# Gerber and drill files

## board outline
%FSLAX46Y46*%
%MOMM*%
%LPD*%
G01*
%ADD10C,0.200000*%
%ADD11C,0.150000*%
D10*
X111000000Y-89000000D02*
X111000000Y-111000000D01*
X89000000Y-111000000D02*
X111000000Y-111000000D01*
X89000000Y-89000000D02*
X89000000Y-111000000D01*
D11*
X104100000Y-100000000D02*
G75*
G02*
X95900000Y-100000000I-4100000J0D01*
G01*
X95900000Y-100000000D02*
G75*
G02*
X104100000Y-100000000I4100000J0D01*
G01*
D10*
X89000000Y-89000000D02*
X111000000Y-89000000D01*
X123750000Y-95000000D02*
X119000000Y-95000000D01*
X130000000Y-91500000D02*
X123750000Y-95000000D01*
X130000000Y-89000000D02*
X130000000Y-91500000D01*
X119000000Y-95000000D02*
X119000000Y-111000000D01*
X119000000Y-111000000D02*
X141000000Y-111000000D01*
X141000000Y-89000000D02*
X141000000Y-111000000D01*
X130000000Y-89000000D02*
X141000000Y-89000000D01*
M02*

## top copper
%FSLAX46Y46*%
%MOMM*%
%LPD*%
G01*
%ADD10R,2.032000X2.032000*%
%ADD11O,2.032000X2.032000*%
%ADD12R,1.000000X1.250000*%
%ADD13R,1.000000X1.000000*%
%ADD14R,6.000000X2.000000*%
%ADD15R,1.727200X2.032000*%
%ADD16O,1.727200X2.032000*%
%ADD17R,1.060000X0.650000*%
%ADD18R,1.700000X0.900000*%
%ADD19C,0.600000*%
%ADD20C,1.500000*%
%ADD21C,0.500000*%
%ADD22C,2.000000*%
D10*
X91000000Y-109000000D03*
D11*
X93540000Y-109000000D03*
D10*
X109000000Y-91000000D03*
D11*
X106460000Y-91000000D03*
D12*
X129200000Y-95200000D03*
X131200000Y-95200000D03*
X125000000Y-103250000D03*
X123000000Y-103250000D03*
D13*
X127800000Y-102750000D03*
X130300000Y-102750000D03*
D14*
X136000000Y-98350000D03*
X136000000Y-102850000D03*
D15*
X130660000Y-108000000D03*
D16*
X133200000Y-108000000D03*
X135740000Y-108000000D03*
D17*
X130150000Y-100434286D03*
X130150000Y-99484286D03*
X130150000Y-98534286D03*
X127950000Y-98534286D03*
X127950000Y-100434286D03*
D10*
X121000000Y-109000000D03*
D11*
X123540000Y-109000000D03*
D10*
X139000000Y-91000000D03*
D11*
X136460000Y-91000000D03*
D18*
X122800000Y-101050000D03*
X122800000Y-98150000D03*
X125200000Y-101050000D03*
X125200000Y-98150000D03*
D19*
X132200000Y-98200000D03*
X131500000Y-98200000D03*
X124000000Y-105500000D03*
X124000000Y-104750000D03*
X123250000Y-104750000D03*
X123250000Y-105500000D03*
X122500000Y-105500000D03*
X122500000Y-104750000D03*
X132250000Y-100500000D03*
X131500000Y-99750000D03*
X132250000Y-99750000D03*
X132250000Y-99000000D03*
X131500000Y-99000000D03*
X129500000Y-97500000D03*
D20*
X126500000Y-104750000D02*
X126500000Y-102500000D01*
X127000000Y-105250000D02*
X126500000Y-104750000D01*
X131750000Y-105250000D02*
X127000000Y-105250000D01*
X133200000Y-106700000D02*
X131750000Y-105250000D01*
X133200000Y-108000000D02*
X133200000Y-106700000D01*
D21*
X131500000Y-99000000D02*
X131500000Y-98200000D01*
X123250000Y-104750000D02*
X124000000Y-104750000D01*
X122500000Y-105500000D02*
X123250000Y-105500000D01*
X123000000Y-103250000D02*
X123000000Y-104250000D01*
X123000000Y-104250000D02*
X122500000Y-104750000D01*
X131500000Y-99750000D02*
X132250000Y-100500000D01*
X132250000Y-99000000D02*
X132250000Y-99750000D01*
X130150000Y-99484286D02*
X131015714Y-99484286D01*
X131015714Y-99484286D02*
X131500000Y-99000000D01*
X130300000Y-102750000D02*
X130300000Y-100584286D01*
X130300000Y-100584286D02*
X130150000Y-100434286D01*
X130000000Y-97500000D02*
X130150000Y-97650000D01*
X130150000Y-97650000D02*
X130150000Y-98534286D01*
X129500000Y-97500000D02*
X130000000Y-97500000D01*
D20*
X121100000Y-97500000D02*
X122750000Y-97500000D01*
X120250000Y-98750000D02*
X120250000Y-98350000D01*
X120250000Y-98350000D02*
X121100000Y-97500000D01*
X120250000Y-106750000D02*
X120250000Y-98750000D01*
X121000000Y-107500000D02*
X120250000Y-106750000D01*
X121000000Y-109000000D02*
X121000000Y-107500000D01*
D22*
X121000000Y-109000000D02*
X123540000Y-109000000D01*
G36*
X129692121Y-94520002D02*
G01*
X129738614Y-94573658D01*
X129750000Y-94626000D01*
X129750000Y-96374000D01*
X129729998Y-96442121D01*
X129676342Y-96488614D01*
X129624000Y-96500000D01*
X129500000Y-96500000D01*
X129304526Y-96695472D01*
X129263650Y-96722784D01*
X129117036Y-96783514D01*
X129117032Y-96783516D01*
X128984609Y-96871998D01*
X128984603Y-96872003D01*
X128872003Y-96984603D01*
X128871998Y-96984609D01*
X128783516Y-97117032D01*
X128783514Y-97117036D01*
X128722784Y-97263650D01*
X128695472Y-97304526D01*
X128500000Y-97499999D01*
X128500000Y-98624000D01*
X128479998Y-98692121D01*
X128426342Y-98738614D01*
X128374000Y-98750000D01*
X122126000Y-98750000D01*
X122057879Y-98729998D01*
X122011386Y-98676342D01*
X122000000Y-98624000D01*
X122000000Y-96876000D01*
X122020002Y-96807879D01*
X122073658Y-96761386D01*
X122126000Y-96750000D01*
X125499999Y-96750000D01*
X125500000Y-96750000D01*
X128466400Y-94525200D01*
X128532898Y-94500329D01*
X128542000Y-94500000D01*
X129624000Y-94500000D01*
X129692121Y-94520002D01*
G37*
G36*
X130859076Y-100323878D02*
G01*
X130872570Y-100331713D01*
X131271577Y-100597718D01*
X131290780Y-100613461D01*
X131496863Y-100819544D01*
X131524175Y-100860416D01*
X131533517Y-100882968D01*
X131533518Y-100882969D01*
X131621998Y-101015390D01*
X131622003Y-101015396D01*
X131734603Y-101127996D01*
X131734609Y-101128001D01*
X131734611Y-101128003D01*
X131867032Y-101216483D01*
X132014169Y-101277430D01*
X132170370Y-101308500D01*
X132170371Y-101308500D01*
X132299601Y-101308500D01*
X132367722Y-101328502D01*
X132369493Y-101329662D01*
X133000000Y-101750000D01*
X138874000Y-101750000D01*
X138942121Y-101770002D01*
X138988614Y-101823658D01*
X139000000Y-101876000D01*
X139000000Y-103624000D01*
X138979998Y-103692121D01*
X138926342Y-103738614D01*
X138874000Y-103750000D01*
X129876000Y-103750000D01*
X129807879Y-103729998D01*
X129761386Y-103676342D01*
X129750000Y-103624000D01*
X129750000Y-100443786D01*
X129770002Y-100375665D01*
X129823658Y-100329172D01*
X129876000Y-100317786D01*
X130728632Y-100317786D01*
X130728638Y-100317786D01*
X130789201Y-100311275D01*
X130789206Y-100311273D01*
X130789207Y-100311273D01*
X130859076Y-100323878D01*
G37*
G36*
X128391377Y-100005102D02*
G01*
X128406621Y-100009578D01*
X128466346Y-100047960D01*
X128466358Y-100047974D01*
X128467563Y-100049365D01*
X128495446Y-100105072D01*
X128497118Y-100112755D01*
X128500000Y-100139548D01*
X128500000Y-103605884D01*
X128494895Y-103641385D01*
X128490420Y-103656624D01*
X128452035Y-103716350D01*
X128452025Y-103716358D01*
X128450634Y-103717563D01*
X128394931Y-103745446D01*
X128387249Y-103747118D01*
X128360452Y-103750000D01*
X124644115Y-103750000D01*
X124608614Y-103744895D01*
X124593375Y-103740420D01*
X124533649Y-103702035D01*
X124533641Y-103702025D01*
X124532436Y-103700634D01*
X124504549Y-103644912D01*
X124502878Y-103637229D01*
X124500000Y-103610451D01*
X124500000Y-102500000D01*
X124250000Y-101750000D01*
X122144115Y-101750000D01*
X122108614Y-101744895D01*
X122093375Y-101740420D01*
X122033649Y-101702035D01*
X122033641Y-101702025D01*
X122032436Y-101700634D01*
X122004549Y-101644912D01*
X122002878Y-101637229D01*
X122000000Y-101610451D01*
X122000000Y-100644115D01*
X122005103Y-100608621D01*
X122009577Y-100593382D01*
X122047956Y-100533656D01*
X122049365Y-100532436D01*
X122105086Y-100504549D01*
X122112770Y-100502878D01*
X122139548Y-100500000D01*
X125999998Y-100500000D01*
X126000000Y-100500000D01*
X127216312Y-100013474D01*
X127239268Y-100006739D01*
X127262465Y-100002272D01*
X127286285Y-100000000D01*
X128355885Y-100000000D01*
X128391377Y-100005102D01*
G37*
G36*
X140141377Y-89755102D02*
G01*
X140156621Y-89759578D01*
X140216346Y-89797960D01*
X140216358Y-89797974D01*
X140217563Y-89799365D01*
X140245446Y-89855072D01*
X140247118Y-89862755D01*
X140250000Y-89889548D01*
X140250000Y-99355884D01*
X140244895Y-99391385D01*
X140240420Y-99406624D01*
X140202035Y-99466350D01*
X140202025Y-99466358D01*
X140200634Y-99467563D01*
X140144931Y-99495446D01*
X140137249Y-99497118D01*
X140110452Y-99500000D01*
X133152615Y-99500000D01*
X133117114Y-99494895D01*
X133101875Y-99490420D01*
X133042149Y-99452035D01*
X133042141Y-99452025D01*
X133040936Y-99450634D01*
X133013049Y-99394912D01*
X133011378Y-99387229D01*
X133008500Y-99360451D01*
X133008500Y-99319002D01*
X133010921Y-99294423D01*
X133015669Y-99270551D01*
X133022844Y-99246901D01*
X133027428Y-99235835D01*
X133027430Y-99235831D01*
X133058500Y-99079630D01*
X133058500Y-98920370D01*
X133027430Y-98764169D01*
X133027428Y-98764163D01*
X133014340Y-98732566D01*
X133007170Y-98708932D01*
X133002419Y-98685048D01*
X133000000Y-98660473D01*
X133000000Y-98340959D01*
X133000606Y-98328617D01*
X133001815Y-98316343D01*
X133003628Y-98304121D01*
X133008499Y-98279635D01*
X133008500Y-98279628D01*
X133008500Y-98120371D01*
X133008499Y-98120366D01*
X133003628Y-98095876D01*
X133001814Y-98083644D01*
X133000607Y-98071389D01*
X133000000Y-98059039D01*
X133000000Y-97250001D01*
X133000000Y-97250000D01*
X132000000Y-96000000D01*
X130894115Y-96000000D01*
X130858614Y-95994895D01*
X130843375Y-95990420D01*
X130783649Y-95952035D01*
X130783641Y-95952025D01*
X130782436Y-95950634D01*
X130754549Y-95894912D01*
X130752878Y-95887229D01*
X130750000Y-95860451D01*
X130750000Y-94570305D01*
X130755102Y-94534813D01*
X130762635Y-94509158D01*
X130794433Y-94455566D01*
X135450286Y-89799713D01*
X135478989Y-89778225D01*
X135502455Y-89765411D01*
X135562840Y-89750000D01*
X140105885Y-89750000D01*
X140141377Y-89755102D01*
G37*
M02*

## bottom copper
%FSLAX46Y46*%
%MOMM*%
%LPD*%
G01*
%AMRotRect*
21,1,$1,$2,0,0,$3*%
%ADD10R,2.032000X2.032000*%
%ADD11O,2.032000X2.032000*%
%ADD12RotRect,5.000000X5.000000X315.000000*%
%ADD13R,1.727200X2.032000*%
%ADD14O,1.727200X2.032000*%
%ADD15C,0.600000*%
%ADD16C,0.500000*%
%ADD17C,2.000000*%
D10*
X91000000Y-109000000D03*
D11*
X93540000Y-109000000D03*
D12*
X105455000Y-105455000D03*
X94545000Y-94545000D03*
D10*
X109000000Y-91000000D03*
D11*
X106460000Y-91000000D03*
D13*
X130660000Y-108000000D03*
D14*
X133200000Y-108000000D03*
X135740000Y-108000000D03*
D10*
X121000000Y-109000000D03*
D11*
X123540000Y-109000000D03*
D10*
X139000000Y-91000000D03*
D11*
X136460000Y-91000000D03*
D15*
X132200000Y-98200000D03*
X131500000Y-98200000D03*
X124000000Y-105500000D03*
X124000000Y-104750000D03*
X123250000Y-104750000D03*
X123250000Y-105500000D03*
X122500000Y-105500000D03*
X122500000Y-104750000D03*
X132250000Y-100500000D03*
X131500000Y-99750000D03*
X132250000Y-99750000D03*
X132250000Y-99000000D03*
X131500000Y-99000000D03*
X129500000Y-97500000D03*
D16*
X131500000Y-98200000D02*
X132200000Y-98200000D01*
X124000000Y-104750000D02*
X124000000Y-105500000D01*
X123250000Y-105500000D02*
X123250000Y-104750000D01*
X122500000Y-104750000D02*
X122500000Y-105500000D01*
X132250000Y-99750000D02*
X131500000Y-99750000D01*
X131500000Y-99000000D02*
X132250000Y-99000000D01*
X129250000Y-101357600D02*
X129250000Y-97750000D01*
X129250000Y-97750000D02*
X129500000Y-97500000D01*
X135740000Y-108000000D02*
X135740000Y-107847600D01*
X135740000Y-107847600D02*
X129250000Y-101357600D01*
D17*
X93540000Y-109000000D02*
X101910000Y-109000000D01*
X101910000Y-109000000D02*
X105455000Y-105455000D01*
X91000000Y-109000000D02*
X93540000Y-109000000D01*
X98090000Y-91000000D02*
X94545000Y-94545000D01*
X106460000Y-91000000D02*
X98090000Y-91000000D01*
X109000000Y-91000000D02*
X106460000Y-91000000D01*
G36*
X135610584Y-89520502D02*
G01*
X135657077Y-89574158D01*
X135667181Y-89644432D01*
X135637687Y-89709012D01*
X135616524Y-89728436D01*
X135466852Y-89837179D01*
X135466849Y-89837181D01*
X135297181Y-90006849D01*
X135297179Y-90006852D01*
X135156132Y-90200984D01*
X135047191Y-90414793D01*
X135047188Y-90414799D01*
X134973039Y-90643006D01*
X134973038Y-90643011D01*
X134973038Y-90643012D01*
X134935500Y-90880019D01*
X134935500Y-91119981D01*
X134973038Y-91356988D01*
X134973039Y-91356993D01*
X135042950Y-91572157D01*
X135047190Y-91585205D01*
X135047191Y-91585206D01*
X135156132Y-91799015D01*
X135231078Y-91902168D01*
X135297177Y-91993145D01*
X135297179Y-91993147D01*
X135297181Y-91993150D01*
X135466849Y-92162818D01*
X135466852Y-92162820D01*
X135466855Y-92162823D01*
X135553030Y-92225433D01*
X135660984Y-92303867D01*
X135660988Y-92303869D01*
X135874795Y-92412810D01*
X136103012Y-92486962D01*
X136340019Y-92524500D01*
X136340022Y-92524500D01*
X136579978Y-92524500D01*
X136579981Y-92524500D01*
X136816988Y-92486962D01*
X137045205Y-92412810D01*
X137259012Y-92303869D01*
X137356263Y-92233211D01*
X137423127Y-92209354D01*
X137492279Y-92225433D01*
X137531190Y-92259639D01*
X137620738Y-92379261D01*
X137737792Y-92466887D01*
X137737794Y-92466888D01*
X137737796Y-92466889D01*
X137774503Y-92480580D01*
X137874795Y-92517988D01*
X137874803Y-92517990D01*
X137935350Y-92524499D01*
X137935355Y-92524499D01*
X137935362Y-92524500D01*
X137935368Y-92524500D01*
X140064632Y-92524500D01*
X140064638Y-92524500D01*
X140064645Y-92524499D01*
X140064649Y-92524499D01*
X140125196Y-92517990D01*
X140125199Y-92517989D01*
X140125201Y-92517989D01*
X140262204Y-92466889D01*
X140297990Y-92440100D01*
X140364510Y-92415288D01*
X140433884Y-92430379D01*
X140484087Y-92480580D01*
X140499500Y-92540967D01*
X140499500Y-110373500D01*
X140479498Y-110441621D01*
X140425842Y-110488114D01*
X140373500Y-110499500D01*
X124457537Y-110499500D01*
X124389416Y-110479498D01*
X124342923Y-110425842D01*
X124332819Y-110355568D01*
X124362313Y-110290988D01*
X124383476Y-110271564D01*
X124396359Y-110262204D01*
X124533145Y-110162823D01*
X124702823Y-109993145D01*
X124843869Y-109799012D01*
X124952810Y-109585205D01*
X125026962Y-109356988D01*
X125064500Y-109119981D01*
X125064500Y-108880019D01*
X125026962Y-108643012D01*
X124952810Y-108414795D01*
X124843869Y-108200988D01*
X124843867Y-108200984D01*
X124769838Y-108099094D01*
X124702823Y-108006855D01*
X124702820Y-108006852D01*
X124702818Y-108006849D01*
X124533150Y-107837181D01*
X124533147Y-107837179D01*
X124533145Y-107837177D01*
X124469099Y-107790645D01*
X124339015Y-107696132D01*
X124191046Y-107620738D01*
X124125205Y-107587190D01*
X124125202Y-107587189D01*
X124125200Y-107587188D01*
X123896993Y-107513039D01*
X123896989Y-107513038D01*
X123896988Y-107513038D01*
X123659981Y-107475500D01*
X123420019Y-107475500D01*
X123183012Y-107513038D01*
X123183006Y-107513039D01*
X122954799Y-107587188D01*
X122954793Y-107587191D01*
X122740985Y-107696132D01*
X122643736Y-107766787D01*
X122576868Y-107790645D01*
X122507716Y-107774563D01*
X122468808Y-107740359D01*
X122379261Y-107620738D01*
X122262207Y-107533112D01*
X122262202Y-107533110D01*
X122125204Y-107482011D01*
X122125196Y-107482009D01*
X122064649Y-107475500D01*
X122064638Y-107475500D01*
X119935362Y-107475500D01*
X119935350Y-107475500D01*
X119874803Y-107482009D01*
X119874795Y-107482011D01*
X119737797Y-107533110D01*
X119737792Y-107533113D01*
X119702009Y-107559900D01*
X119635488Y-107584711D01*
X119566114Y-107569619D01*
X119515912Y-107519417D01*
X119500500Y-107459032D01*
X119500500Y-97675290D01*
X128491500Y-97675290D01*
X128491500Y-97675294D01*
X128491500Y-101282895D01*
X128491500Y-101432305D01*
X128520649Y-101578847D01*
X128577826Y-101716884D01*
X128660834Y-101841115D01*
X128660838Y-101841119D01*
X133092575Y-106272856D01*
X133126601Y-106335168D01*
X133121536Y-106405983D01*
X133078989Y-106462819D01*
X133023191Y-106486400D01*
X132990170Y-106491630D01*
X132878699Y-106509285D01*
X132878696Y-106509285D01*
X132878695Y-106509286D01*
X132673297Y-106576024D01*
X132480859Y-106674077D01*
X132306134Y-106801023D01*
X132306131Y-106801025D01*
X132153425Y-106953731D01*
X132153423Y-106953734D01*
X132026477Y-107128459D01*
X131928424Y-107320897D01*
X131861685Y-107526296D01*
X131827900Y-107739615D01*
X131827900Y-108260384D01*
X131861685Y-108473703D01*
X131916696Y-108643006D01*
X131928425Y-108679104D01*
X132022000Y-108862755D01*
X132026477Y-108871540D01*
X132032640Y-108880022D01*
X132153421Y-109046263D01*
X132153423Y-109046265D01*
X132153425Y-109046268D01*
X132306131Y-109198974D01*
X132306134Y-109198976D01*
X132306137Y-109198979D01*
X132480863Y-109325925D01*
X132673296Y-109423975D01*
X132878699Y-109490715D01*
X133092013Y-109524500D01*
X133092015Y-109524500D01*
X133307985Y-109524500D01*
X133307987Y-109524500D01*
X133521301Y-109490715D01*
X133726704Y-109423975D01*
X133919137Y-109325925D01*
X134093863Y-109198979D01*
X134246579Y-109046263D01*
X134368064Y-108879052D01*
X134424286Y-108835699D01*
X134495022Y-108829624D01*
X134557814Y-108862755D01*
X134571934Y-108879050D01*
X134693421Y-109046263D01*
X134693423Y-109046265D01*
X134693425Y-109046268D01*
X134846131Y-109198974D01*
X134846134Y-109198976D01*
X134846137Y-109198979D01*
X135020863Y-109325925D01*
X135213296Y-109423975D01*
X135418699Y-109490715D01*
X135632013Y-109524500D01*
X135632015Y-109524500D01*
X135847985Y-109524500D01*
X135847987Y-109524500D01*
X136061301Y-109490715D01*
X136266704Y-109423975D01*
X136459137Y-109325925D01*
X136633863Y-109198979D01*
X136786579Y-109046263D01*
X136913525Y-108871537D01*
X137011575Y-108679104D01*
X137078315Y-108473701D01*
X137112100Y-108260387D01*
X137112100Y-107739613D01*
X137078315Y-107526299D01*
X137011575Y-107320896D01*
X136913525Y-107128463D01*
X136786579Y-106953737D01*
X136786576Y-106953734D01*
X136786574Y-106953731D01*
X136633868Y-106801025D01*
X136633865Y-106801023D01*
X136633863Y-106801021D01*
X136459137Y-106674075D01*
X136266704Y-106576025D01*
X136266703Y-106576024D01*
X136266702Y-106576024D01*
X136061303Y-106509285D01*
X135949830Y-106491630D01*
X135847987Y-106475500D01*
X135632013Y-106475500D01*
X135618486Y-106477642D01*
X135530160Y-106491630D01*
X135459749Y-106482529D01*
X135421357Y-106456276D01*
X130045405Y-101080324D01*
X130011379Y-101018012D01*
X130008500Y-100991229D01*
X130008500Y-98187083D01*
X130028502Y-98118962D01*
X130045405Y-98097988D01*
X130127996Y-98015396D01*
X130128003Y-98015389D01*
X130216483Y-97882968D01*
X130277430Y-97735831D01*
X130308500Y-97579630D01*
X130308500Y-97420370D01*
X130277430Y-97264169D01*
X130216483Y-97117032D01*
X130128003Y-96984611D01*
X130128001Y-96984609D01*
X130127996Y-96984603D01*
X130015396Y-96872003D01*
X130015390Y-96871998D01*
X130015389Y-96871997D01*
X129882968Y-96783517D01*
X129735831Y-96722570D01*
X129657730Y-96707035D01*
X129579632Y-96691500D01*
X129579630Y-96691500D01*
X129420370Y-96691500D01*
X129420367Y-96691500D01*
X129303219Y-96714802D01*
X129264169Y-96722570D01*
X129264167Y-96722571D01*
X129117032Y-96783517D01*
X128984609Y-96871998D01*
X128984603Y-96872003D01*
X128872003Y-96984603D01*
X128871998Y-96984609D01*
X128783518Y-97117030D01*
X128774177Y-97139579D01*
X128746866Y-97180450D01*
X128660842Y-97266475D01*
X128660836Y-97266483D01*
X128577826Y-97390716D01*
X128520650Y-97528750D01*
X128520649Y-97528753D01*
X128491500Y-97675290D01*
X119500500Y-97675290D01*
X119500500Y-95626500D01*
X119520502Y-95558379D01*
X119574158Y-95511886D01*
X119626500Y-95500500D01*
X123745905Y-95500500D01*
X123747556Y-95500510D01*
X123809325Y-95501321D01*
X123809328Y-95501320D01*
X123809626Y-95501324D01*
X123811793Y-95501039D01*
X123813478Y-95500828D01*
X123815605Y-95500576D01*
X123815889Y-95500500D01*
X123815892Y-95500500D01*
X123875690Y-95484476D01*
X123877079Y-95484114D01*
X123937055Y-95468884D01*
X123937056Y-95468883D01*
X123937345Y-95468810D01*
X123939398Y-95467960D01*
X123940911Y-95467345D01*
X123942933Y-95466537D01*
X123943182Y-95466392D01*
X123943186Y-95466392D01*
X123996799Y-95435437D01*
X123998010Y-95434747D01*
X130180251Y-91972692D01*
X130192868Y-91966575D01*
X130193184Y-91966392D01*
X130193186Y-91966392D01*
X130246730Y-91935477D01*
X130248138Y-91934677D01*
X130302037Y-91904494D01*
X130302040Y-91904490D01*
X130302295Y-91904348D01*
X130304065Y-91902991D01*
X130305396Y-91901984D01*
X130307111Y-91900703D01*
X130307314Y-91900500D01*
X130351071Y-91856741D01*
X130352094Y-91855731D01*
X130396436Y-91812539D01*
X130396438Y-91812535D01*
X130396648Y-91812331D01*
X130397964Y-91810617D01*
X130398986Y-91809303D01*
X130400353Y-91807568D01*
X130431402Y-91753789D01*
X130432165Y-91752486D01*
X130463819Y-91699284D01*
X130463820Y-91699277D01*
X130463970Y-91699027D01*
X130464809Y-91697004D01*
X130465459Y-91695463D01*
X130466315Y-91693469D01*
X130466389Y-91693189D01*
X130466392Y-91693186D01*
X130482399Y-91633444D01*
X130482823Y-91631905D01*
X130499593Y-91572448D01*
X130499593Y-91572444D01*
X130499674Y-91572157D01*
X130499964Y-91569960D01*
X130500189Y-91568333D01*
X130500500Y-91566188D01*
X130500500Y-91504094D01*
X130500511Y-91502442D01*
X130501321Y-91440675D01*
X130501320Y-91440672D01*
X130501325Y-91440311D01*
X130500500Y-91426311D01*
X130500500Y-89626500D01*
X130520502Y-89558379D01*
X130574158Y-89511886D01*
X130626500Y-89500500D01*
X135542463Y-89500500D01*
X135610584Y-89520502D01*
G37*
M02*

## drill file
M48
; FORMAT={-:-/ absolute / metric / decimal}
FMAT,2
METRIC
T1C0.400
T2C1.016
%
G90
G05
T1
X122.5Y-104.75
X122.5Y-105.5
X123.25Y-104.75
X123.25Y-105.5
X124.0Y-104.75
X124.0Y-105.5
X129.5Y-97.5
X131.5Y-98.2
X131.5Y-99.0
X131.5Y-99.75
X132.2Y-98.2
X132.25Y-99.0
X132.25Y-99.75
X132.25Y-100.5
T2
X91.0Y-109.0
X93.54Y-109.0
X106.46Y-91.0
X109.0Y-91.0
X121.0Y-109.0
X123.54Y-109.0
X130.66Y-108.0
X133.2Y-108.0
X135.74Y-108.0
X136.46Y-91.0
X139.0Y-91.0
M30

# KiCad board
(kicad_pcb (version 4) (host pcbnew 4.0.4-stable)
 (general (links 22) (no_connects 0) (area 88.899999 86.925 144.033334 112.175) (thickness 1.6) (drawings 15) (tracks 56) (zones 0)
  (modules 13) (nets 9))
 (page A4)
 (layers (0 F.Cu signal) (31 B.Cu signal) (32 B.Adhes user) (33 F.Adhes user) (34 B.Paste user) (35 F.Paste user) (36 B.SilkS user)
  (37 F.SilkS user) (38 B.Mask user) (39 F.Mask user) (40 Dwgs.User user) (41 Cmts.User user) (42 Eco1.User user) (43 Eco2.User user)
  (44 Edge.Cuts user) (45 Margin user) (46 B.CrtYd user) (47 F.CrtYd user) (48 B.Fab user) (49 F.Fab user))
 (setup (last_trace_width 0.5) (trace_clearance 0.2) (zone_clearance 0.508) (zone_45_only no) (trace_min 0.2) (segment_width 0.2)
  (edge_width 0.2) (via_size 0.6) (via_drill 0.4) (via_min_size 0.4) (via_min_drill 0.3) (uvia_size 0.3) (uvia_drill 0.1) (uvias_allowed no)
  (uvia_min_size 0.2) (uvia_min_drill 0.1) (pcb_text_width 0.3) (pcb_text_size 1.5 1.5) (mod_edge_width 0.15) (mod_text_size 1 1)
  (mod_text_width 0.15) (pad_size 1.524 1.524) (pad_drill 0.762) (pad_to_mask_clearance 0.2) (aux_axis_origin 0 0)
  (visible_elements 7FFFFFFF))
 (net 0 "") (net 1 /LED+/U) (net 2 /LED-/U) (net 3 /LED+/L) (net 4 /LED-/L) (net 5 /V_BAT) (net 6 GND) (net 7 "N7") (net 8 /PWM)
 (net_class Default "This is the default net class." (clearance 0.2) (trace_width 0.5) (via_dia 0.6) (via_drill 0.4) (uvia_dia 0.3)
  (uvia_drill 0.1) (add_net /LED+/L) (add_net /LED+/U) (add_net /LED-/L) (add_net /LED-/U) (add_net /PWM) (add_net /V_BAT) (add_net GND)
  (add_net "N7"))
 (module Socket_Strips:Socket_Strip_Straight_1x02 (layer B.Cu) (at 91 109)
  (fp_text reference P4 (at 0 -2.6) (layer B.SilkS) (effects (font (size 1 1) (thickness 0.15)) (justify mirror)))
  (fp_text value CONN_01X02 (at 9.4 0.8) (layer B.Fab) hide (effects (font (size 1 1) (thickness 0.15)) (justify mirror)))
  (pad 1 thru_hole rect (at 0 0) (size 2.032 2.032) (drill 1.016) (layers *.Cu *.Mask) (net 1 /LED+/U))
  (pad 2 thru_hole oval (at 2.54 0) (size 2.032 2.032) (drill 1.016) (layers *.Cu *.Mask) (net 1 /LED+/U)))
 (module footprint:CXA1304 (layer B.Cu) (at 100 100)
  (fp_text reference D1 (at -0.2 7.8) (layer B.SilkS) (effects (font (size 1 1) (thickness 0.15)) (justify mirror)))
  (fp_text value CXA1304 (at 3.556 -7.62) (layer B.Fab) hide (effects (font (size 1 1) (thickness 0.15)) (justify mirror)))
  (pad 2 smd rect (at 5.455 5.455 315) (size 5 5) (layers B.Cu B.Paste B.Mask) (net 1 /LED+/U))
  (pad 1 smd rect (at -5.455 -5.455 315) (size 5 5) (layers B.Cu B.Paste B.Mask) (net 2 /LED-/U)))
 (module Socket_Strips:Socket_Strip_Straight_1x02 (layer B.Cu) (at 109 91 180)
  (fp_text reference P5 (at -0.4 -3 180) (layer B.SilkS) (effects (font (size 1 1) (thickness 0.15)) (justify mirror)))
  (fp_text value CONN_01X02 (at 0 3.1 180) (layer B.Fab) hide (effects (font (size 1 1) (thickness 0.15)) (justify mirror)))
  (pad 1 thru_hole rect (at 0 0 180) (size 2.032 2.032) (drill 1.016) (layers *.Cu *.Mask) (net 2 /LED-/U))
  (pad 2 thru_hole oval (at 2.54 0 180) (size 2.032 2.032) (drill 1.016) (layers *.Cu *.Mask) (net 2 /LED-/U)))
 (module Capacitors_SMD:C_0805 (layer F.Cu) (at 130.2 95.2)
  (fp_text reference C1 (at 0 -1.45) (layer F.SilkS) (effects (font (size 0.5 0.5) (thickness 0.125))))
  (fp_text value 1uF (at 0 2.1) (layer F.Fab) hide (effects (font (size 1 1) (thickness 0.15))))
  (pad 1 smd rect (at -1 0) (size 1 1.25) (layers F.Cu F.Paste F.Mask) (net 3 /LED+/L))
  (pad 2 smd rect (at 1 0) (size 1 1.25) (layers F.Cu F.Paste F.Mask) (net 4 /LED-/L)))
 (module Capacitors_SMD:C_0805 (layer F.Cu) (at 124 103.25 180)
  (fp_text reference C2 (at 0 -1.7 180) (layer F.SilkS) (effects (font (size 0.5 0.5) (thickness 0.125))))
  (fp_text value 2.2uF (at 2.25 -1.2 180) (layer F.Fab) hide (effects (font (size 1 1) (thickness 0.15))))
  (pad 1 smd rect (at -1 0 180) (size 1 1.25) (layers F.Cu F.Paste F.Mask) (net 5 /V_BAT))
  (pad 2 smd rect (at 1 0 180) (size 1 1.25) (layers F.Cu F.Paste F.Mask) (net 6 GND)))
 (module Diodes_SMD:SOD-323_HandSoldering (layer F.Cu) (at 129.05 102.75)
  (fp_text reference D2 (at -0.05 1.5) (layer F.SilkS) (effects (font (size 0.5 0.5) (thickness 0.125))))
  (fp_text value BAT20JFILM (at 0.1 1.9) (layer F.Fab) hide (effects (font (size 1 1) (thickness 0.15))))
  (pad 1 smd rect (at -1.25 0) (size 1 1) (layers F.Cu F.Paste F.Mask) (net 5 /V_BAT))
  (pad 2 smd rect (at 1.25 0) (size 1 1) (layers F.Cu F.Paste F.Mask) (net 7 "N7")))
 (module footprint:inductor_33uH (layer F.Cu) (at 136 100.6 270)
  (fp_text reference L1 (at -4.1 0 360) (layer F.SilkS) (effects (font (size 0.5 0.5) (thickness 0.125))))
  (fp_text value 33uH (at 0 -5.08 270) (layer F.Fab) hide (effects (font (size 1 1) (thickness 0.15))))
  (pad 1 smd rect (at -2.25 0 270) (size 2 6) (layers F.Cu F.Paste F.Mask) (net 4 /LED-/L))
  (pad 2 smd rect (at 2.25 0 270) (size 2 6) (layers F.Cu F.Paste F.Mask) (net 7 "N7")))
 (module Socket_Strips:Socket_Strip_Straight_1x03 (layer B.Cu) (at 130.66 108)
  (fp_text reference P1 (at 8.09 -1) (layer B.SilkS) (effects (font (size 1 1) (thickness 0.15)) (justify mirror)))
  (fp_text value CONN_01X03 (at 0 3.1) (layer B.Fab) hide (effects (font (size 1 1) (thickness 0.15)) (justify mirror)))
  (pad 1 thru_hole rect (at 0 0) (size 1.7272 2.032) (drill 1.016) (layers *.Cu *.Mask) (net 6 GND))
  (pad 2 thru_hole oval (at 2.54 0) (size 1.7272 2.032) (drill 1.016) (layers *.Cu *.Mask) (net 5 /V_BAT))
  (pad 3 thru_hole oval (at 5.08 0) (size 1.7272 2.032) (drill 1.016) (layers *.Cu *.Mask) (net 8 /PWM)))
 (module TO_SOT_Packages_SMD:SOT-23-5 (layer F.Cu) (at 129.05 99.484286 180)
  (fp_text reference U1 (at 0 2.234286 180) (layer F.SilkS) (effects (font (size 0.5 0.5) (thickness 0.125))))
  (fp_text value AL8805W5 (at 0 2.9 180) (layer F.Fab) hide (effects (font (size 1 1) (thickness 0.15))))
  (pad 1 smd rect (at -1.1 -0.95 180) (size 1.06 0.65) (layers F.Cu F.Paste F.Mask) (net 7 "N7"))
  (pad 2 smd rect (at -1.1 0 180) (size 1.06 0.65) (layers F.Cu F.Paste F.Mask) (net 6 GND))
  (pad 3 smd rect (at -1.1 0.95 180) (size 1.06 0.65) (layers F.Cu F.Paste F.Mask) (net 8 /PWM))
  (pad 4 smd rect (at 1.1 0.95 180) (size 1.06 0.65) (layers F.Cu F.Paste F.Mask) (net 3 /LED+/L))
  (pad 5 smd rect (at 1.1 -0.95 180) (size 1.06 0.65) (layers F.Cu F.Paste F.Mask) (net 5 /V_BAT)))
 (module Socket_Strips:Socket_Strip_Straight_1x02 (layer F.Cu) (at 121 109)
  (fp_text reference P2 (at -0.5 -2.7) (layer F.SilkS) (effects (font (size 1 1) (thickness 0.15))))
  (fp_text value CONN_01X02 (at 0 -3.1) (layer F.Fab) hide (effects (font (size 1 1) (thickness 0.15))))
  (pad 1 thru_hole rect (at 0 0) (size 2.032 2.032) (drill 1.016) (layers *.Cu *.Mask) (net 3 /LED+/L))
  (pad 2 thru_hole oval (at 2.54 0) (size 2.032 2.032) (drill 1.016) (layers *.Cu *.Mask) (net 3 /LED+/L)))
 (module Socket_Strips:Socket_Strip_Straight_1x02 (layer F.Cu) (at 139 91 180)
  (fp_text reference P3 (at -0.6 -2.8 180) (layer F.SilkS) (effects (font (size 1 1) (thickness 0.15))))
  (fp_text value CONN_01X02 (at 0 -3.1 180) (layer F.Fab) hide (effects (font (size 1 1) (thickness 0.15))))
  (pad 1 thru_hole rect (at 0 0 180) (size 2.032 2.032) (drill 1.016) (layers *.Cu *.Mask) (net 4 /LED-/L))
  (pad 2 thru_hole oval (at 2.54 0 180) (size 2.032 2.032) (drill 1.016) (layers *.Cu *.Mask) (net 4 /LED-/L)))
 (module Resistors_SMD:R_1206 (layer F.Cu) (at 122.8 99.6 90)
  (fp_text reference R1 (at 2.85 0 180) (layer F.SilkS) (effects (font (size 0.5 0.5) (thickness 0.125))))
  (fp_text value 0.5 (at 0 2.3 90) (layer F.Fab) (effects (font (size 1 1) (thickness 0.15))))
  (pad 1 smd rect (at -1.45 0 90) (size 0.9 1.7) (layers F.Cu F.Paste F.Mask) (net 5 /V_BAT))
  (pad 2 smd rect (at 1.45 0 90) (size 0.9 1.7) (layers F.Cu F.Paste F.Mask) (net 3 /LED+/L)))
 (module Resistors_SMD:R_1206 (layer F.Cu) (at 125.2 99.6 90)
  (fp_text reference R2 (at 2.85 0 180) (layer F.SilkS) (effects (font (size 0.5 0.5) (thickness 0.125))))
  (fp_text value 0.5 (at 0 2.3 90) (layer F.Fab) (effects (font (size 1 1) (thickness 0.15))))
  (pad 1 smd rect (at -1.45 0 90) (size 0.9 1.7) (layers F.Cu F.Paste F.Mask) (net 5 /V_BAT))
  (pad 2 smd rect (at 1.45 0 90) (size 0.9 1.7) (layers F.Cu F.Paste F.Mask) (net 3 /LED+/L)))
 (gr_line (start 111 89) (end 111 111) (layer Edge.Cuts) (width 0.2))
 (gr_line (start 89 111) (end 111 111) (layer Edge.Cuts) (width 0.2))
 (gr_line (start 89 89) (end 89 111) (layer Edge.Cuts) (width 0.2))
 (gr_circle (center 100 100) (end 100 95.9) (layer Edge.Cuts) (width 0.15))
 (gr_line (start 89 89) (end 111 89) (layer Edge.Cuts) (width 0.2))
 (gr_line (start 123.75 95) (end 119 95) (layer Edge.Cuts) (width 0.2))
 (gr_line (start 130 91.5) (end 123.75 95) (layer Edge.Cuts) (width 0.2))
 (gr_line (start 130 89) (end 130 91.5) (layer Edge.Cuts) (width 0.2))
 (gr_line (start 119 95) (end 119 111) (layer Edge.Cuts) (width 0.2))
 (gr_line (start 119 111) (end 141 111) (layer Edge.Cuts) (width 0.2))
 (gr_line (start 141 89) (end 141 111) (layer Edge.Cuts) (width 0.2))
 (gr_line (start 130 89) (end 141 89) (layer Edge.Cuts) (width 0.2))
 (segment (start 126.5 104.75) (end 126.5 102.5) (width 1.5) (layer F.Cu) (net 5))
 (segment (start 127 105.25) (end 126.5 104.75) (width 1.5) (layer F.Cu) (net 5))
 (segment (start 131.75 105.25) (end 127 105.25) (width 1.5) (layer F.Cu) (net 5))
 (segment (start 133.2 106.7) (end 131.75 105.25) (width 1.5) (layer F.Cu) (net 5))
 (segment (start 133.2 108) (end 133.2 106.7) (width 1.5) (layer F.Cu) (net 5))
 (segment (start 131.5 98.2) (end 132.2 98.2) (width 0.5) (layer B.Cu) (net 6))
 (via (at 132.2 98.2) (size 0.6) (drill 0.4) (layers F.Cu B.Cu) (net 6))
 (segment (start 131.5 99) (end 131.5 98.2) (width 0.5) (layer F.Cu) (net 6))
 (via (at 131.5 98.2) (size 0.6) (drill 0.4) (layers F.Cu B.Cu) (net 6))
 (segment (start 124 104.75) (end 124 105.5) (width 0.5) (layer B.Cu) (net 6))
 (via (at 124 105.5) (size 0.6) (drill 0.4) (layers F.Cu B.Cu) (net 6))
 (segment (start 123.25 104.75) (end 124 104.75) (width 0.5) (layer F.Cu) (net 6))
 (via (at 124 104.75) (size 0.6) (drill 0.4) (layers F.Cu B.Cu) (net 6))
 (segment (start 123.25 105.5) (end 123.25 104.75) (width 0.5) (layer B.Cu) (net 6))
 (via (at 123.25 104.75) (size 0.6) (drill 0.4) (layers F.Cu B.Cu) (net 6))
 (segment (start 122.5 105.5) (end 123.25 105.5) (width 0.5) (layer F.Cu) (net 6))
 (via (at 123.25 105.5) (size 0.6) (drill 0.4) (layers F.Cu B.Cu) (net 6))
 (segment (start 122.5 104.75) (end 122.5 105.5) (width 0.5) (layer B.Cu) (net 6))
 (via (at 122.5 105.5) (size 0.6) (drill 0.4) (layers F.Cu B.Cu) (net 6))
 (segment (start 123 103.25) (end 123 104.25) (width 0.5) (layer F.Cu) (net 6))
 (segment (start 123 104.25) (end 122.5 104.75) (width 0.5) (layer F.Cu) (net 6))
 (via (at 122.5 104.75) (size 0.6) (drill 0.4) (layers F.Cu B.Cu) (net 6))
 (segment (start 131.5 99.75) (end 132.25 100.5) (width 0.5) (layer F.Cu) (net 6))
 (via (at 132.25 100.5) (size 0.6) (drill 0.4) (layers F.Cu B.Cu) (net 6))
 (segment (start 132.25 99.75) (end 131.5 99.75) (width 0.5) (layer B.Cu) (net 6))
 (via (at 131.5 99.75) (size 0.6) (drill 0.4) (layers F.Cu B.Cu) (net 6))
 (segment (start 132.25 99) (end 132.25 99.75) (width 0.5) (layer F.Cu) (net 6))
 (via (at 132.25 99.75) (size 0.6) (drill 0.4) (layers F.Cu B.Cu) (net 6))
 (segment (start 131.5 99) (end 132.25 99) (width 0.5) (layer B.Cu) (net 6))
 (via (at 132.25 99) (size 0.6) (drill 0.4) (layers F.Cu B.Cu) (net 6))
 (segment (start 130.15 99.484286) (end 131.015714 99.484286) (width 0.5) (layer F.Cu) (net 6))
 (segment (start 131.015714 99.484286) (end 131.5 99) (width 0.5) (layer F.Cu) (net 6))
 (via (at 131.5 99) (size 0.6) (drill 0.4) (layers F.Cu B.Cu) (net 6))
 (segment (start 130.3 102.75) (end 130.3 100.584286) (width 0.5) (layer F.Cu) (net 7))
 (segment (start 130.3 100.584286) (end 130.15 100.434286) (width 0.5) (layer F.Cu) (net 7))
 (segment (start 130 97.5) (end 130.15 97.65) (width 0.5) (layer F.Cu) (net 8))
 (segment (start 130.15 97.65) (end 130.15 98.534286) (width 0.5) (layer F.Cu) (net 8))
 (segment (start 129.5 97.5) (end 130 97.5) (width 0.5) (layer F.Cu) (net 8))
 (segment (start 129.25 101.3576) (end 129.25 97.75) (width 0.5) (layer B.Cu) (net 8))
 (segment (start 129.25 97.75) (end 129.5 97.5) (width 0.5) (layer B.Cu) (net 8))
 (via (at 129.5 97.5) (size 0.6) (drill 0.4) (layers F.Cu B.Cu) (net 8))
 (segment (start 135.74 108) (end 135.74 107.8476) (width 0.5) (layer B.Cu) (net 8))
 (segment (start 135.74 107.8476) (end 129.25 101.3576) (width 0.5) (layer B.Cu) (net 8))
 (segment (start 121.1 97.5) (end 122.75 97.5) (width 1.5) (layer F.Cu) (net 3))
 (segment (start 120.25 98.75) (end 120.25 98.35) (width 1.5) (layer F.Cu) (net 3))
 (segment (start 120.25 98.35) (end 121.1 97.5) (width 1.5) (layer F.Cu) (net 3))
 (segment (start 120.25 106.75) (end 120.25 98.75) (width 1.5) (layer F.Cu) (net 3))
 (segment (start 121 107.5) (end 120.25 106.75) (width 1.5) (layer F.Cu) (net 3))
 (segment (start 121 109) (end 121 107.5) (width 1.5) (layer F.Cu) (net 3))
 (segment (start 121 109) (end 123.54 109) (width 2) (layer F.Cu) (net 3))
 (segment (start 93.54 109) (end 101.91 109) (width 2) (layer B.Cu) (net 1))
 (segment (start 101.91 109) (end 105.455 105.455) (width 2) (layer B.Cu) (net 1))
 (segment (start 91 109) (end 93.54 109) (width 2) (layer B.Cu) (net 1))
 (segment (start 98.09 91) (end 94.545 94.545) (width 2) (layer B.Cu) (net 2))
 (segment (start 106.46 91) (end 98.09 91) (width 2) (layer B.Cu) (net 2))
 (segment (start 109 91) (end 106.46 91) (width 2) (layer B.Cu) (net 2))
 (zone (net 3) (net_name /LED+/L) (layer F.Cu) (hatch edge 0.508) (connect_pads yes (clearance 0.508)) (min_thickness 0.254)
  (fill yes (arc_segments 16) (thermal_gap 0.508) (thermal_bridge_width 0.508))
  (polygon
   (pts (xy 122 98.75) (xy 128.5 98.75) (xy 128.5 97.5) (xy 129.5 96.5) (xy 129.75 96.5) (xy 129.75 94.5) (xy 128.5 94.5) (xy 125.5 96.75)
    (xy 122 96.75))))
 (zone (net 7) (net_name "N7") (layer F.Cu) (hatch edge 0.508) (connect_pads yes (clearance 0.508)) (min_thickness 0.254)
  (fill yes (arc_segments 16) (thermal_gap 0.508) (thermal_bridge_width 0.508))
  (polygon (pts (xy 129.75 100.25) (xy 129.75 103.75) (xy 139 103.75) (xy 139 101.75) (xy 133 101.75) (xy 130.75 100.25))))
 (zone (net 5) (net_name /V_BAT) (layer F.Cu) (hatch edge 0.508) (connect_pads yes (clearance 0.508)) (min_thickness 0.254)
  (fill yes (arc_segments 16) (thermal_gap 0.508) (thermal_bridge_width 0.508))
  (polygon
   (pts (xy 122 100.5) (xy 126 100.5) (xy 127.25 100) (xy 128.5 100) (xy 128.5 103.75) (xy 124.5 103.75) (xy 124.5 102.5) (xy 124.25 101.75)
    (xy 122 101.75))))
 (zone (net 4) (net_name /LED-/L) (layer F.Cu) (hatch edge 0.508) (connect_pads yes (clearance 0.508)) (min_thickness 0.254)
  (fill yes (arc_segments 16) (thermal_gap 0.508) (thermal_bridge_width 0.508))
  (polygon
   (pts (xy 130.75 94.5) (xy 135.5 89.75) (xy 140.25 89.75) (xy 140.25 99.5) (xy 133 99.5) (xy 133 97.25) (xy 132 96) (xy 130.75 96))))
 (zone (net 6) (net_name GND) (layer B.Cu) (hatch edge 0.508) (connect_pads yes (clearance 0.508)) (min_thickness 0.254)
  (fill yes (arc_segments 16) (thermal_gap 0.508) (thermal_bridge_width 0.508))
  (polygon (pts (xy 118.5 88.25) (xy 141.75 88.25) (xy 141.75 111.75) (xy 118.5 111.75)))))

